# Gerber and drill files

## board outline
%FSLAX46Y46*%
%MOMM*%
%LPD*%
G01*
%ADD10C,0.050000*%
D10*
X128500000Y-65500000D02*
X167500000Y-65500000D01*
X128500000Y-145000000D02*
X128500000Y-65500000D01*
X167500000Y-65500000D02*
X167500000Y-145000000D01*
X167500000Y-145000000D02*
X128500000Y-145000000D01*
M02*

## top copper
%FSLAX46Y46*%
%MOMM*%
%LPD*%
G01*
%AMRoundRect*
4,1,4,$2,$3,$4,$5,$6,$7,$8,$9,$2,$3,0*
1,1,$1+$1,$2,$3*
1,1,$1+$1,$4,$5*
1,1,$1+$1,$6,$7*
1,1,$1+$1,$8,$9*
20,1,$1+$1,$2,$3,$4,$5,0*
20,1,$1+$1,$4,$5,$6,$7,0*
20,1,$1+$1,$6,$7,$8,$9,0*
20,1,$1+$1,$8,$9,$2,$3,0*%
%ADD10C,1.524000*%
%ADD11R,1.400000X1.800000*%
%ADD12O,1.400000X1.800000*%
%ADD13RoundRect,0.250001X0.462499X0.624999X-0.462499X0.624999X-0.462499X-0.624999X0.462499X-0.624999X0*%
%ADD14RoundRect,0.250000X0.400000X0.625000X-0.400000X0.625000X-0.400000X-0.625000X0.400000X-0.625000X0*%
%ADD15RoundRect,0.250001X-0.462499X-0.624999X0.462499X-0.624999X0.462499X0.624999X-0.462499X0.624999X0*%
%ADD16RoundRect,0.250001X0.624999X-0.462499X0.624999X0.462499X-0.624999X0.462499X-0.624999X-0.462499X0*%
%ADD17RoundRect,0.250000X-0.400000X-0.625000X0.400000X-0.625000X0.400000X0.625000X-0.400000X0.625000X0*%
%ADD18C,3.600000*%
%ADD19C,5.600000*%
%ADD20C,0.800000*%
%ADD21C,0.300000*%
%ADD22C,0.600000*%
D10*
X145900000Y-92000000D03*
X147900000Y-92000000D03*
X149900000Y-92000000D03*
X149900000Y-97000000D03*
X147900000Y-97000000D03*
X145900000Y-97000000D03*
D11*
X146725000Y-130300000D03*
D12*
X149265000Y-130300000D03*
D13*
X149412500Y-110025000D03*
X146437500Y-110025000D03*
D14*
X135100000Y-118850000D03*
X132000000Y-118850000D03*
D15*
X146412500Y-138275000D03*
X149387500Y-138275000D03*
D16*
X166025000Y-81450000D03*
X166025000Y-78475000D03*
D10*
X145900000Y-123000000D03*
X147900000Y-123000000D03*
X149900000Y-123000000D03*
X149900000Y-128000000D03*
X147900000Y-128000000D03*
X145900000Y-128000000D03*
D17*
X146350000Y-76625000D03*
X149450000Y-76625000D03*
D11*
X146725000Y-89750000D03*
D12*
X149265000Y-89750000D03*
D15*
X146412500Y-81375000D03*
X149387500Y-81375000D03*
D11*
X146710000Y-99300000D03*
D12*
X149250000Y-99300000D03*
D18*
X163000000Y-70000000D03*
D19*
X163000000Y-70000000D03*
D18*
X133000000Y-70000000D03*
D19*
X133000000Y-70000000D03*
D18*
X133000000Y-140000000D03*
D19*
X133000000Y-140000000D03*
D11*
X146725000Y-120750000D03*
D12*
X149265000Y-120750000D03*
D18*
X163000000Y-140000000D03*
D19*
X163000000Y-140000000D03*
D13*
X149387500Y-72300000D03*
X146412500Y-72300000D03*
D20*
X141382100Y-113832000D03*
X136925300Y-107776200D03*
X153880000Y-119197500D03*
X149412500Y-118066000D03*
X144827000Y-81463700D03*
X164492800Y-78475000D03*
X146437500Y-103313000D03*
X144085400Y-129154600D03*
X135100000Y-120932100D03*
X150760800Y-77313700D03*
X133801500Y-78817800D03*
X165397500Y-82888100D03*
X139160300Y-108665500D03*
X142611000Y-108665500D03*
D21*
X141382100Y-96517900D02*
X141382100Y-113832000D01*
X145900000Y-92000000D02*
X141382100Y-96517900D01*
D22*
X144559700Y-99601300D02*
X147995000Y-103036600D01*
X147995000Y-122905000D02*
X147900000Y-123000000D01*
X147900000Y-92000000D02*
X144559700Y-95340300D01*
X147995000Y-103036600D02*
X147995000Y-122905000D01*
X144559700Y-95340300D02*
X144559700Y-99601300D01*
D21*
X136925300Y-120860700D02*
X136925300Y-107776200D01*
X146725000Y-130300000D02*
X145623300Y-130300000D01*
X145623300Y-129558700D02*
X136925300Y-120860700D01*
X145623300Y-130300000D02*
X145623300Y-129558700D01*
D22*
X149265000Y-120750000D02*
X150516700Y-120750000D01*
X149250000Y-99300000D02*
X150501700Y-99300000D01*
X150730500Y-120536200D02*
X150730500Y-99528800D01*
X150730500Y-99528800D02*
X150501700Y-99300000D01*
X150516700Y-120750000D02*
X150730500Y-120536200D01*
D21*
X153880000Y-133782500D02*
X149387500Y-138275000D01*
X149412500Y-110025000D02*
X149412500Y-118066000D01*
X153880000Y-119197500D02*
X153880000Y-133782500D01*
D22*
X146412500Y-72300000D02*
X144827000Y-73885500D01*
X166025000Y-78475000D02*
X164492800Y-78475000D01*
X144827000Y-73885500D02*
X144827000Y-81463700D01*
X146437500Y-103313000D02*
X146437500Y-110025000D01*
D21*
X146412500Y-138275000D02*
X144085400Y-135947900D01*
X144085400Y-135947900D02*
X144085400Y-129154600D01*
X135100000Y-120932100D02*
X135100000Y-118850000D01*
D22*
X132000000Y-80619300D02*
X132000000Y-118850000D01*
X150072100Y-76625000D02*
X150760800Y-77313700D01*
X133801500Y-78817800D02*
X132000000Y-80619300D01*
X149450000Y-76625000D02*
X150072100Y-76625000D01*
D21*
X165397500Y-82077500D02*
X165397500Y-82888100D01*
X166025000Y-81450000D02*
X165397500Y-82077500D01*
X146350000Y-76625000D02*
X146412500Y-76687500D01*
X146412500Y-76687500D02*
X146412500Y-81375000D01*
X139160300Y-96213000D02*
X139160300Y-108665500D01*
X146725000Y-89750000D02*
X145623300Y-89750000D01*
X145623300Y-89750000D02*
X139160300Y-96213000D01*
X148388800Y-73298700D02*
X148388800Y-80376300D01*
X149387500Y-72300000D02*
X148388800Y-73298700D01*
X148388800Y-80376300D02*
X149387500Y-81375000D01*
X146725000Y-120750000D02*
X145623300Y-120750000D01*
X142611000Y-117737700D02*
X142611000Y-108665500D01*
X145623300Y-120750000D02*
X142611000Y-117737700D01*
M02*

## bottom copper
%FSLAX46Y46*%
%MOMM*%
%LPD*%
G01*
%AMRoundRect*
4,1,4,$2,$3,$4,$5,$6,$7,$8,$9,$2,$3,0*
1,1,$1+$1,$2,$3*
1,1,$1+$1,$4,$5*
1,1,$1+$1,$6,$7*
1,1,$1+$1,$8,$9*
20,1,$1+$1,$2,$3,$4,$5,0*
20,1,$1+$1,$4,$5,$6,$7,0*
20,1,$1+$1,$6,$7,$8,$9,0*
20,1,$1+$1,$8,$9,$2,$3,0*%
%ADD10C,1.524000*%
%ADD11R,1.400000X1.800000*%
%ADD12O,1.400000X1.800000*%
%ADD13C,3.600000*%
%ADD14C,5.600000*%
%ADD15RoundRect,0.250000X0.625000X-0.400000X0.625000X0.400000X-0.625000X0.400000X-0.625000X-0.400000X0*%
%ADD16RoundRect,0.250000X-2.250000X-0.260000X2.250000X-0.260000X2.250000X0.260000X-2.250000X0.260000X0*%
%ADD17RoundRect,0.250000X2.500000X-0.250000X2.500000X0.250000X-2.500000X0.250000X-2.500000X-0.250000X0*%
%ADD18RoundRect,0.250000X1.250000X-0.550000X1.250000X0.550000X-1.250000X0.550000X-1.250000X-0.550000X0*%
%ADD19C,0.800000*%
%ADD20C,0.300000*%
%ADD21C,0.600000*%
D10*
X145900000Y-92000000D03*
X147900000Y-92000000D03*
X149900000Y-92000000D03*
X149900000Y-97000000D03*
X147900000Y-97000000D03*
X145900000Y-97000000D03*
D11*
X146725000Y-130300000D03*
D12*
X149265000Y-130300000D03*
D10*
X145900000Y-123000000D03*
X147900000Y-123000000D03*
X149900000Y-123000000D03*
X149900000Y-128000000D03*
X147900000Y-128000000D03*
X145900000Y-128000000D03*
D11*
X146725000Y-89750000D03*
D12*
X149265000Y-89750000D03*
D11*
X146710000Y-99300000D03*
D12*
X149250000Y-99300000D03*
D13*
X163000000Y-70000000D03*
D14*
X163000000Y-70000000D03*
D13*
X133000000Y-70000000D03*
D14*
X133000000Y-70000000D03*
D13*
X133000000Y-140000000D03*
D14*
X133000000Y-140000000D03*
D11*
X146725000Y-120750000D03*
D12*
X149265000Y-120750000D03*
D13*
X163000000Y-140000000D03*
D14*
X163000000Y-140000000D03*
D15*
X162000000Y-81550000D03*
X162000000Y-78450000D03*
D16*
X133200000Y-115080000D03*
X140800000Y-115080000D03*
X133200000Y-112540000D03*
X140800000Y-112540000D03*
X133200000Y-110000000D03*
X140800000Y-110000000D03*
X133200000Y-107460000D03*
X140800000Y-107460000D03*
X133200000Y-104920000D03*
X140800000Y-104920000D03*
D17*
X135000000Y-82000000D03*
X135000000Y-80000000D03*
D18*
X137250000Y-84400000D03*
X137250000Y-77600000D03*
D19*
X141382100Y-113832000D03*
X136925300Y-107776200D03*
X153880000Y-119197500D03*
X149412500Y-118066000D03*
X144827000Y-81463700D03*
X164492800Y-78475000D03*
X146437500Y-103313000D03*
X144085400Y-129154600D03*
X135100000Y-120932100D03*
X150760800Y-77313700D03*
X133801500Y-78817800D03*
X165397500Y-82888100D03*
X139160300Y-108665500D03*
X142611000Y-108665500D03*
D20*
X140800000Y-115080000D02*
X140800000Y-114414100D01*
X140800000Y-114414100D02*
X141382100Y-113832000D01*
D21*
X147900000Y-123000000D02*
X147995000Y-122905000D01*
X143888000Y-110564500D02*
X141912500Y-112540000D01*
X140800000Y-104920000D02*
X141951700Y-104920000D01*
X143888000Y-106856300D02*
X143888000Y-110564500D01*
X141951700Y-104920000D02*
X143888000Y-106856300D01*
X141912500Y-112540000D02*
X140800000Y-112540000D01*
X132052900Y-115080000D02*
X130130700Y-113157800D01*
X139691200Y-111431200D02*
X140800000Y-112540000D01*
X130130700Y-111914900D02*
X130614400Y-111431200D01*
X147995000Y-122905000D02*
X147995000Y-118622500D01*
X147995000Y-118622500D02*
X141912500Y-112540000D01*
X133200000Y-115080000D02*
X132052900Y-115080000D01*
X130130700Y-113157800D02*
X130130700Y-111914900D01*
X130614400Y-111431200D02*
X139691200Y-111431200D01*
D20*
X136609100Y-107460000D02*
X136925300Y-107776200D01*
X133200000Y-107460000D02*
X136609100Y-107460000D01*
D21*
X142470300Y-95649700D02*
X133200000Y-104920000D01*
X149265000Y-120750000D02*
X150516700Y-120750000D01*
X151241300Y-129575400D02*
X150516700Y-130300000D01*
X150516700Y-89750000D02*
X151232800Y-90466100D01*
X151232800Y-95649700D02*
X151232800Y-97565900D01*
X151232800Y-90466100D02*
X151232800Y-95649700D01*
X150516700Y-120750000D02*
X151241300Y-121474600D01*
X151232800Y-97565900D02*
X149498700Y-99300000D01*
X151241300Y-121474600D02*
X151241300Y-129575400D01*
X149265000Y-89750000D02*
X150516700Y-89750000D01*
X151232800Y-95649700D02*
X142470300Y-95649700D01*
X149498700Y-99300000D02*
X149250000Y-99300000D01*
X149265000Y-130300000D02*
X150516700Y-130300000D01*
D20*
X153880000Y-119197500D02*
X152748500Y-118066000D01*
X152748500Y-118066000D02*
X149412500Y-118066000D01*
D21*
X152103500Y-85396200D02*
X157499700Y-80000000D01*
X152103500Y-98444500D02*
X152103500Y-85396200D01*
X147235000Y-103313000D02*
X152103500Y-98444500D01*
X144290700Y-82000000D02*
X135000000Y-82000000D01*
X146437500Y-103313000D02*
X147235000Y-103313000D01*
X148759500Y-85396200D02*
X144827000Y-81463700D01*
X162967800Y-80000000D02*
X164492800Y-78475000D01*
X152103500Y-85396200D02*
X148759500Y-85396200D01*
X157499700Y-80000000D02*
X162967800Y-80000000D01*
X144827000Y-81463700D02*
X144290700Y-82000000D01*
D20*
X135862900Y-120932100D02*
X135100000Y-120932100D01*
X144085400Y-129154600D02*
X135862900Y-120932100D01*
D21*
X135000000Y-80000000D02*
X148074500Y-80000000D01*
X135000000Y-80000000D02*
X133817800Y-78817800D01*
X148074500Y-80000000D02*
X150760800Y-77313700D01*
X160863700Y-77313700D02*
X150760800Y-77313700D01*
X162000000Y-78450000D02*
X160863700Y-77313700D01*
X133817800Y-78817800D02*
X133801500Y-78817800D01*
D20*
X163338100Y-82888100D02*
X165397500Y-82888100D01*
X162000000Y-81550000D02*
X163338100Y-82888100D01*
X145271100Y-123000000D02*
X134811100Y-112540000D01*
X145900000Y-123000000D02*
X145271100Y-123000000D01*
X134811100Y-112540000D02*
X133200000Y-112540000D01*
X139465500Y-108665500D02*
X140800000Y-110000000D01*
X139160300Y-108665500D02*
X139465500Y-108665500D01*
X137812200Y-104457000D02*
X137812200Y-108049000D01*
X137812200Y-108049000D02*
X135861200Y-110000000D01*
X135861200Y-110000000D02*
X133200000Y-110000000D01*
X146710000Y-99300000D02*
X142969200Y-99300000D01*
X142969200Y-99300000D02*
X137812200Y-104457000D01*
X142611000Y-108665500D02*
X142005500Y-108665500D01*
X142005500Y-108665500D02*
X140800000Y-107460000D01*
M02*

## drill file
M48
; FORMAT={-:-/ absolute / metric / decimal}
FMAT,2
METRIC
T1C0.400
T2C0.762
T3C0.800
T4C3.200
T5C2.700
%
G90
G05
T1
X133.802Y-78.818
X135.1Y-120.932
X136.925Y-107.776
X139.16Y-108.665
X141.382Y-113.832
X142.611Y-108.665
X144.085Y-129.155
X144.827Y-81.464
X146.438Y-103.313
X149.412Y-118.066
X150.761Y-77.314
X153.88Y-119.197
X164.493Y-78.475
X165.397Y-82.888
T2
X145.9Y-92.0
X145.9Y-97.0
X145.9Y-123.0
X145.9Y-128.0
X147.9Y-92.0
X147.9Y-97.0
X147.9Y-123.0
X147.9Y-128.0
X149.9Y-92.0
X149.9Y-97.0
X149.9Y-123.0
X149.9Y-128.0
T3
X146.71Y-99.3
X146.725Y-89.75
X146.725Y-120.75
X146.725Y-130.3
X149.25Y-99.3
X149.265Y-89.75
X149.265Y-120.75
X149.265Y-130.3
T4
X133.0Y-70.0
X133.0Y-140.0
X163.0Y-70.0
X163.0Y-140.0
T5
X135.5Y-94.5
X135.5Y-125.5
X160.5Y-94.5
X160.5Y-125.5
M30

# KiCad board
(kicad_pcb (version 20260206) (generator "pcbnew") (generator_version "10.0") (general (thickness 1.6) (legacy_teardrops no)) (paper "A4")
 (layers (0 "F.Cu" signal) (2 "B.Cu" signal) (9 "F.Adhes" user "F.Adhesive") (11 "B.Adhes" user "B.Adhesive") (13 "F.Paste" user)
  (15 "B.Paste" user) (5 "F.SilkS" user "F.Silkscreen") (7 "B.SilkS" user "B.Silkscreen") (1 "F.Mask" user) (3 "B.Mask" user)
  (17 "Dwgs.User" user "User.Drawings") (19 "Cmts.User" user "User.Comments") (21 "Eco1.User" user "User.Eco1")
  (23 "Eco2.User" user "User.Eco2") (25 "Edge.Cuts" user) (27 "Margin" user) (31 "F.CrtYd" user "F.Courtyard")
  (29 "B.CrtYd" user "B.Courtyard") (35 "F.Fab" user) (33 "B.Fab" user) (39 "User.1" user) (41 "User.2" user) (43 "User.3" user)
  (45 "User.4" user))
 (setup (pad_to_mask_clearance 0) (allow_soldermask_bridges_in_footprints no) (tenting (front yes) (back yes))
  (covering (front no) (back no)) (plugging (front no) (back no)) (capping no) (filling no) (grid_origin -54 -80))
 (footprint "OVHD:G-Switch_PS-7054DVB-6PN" (layer "F.Cu") (at 148.5 100)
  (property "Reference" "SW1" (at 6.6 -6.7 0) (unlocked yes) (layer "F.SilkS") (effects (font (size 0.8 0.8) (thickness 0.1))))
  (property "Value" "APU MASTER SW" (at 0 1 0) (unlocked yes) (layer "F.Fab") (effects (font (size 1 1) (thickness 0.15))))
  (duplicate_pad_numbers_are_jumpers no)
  (pad "1" thru_hole circle (at -2.6 -8) (size 1.524 1.524) (drill 0.762) (layers "*.Cu" "*.Mask") (remove_unused_layers no)
   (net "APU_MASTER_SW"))
  (pad "2" thru_hole circle (at -0.6 -8) (size 1.524 1.524) (drill 0.762) (layers "*.Cu" "*.Mask") (remove_unused_layers no) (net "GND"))
  (pad "3" thru_hole circle (at 1.4 -8) (size 1.524 1.524) (drill 0.762) (layers "*.Cu" "*.Mask") (remove_unused_layers no)
   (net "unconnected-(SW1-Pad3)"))
  (pad "4" thru_hole circle (at 1.4 -3) (size 1.524 1.524) (drill 0.762) (layers "*.Cu" "*.Mask") (remove_unused_layers no)
   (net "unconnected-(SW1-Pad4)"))
  (pad "5" thru_hole circle (at -0.6 -3) (size 1.524 1.524) (drill 0.762) (layers "*.Cu" "*.Mask") (remove_unused_layers no)
   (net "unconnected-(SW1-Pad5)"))
  (pad "6" thru_hole circle (at -2.6 -3) (size 1.524 1.524) (drill 0.762) (layers "*.Cu" "*.Mask") (remove_unused_layers no)
   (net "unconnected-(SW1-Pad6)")))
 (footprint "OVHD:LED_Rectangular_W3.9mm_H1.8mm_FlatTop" (layer "F.Cu") (at 146.725 130.3)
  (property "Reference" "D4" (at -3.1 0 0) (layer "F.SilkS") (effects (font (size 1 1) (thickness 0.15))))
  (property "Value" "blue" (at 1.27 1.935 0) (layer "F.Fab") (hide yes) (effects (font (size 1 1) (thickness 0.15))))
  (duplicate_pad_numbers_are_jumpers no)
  (pad "1" thru_hole rect (at 0 0) (size 1.4 1.8) (drill 0.8) (layers "*.Cu" "*.Mask") (remove_unused_layers no) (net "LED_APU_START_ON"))
  (pad "2" thru_hole oval (at 2.54 0) (size 1.4 1.8) (drill 0.8) (layers "*.Cu" "*.Mask") (remove_unused_layers no) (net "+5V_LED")))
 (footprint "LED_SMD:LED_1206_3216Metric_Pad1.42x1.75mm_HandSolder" (layer "F.Cu") (at 147.925 110.025 180)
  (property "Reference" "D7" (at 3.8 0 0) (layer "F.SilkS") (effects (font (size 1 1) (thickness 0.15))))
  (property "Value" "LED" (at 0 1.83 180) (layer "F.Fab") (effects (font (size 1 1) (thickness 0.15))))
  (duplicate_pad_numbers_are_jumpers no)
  (pad "1" smd roundrect (at -1.4875 0 180) (size 1.425 1.75) (layers "F.Cu" "F.Mask" "F.Paste") (roundrect_rratio 0.175439) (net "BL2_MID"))
  (pad "2" smd roundrect (at 1.4875 0 180) (size 1.425 1.75) (layers "F.Cu" "F.Mask" "F.Paste") (roundrect_rratio 0.175439) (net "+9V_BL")))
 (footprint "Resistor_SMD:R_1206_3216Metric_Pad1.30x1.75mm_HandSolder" (layer "F.Cu") (at 133.55 118.85 180)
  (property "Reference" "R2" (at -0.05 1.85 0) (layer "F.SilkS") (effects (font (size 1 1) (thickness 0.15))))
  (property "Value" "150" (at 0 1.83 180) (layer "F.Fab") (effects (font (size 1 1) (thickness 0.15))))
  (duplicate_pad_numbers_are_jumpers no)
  (pad "1" smd roundrect (at -1.55 0 180) (size 1.3 1.75) (layers "F.Cu" "F.Mask" "F.Paste") (roundrect_rratio 0.192308) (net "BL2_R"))
  (pad "2" smd roundrect (at 1.55 0 180) (size 1.3 1.75) (layers "F.Cu" "F.Mask" "F.Paste") (roundrect_rratio 0.192308) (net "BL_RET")))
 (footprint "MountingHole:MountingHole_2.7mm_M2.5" (layer "F.Cu") (at 135.5 125.5)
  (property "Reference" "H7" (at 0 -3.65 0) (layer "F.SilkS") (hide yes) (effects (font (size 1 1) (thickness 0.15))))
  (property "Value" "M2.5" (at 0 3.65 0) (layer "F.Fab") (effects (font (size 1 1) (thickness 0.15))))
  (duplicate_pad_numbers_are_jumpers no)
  (pad "" np_thru_hole circle (at 0 0) (size 2.7 2.7) (drill 2.7) (layers "*.Cu" "*.Mask")))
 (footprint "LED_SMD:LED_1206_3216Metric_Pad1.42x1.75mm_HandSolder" (layer "F.Cu") (at 147.9 138.275)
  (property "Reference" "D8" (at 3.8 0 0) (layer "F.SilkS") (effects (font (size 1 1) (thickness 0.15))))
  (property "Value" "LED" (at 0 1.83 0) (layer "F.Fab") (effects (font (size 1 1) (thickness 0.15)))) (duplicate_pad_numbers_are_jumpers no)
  (pad "1" smd roundrect (at -1.4875 0) (size 1.425 1.75) (layers "F.Cu" "F.Mask" "F.Paste") (roundrect_rratio 0.175439) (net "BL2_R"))
  (pad "2" smd roundrect (at 1.4875 0) (size 1.425 1.75) (layers "F.Cu" "F.Mask" "F.Paste") (roundrect_rratio 0.175439) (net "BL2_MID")))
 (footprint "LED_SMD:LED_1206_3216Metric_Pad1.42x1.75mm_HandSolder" (layer "F.Cu") (at 166.025 79.9625 90)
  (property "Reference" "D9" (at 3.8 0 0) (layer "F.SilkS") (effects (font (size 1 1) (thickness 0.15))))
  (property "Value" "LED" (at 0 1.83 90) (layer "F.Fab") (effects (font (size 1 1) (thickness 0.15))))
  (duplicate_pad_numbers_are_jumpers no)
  (pad "1" smd roundrect (at -1.4875 0 90) (size 1.425 1.75) (layers "F.Cu" "F.Mask" "F.Paste") (roundrect_rratio 0.175439) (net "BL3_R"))
  (pad "2" smd roundrect (at 1.4875 0 90) (size 1.425 1.75) (layers "F.Cu" "F.Mask" "F.Paste") (roundrect_rratio 0.175439) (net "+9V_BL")))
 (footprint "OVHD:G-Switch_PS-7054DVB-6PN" (layer "F.Cu") (at 148.5 131)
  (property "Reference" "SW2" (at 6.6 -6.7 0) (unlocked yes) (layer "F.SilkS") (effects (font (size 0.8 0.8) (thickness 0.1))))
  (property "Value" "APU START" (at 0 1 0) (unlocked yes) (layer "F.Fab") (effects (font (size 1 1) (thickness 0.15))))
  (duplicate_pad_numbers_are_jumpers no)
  (pad "1" thru_hole circle (at -2.6 -8) (size 1.524 1.524) (drill 0.762) (layers "*.Cu" "*.Mask") (remove_unused_layers no)
   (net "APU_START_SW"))
  (pad "2" thru_hole circle (at -0.6 -8) (size 1.524 1.524) (drill 0.762) (layers "*.Cu" "*.Mask") (remove_unused_layers no) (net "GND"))
  (pad "3" thru_hole circle (at 1.4 -8) (size 1.524 1.524) (drill 0.762) (layers "*.Cu" "*.Mask") (remove_unused_layers no)
   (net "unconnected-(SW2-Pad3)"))
  (pad "4" thru_hole circle (at 1.4 -3) (size 1.524 1.524) (drill 0.762) (layers "*.Cu" "*.Mask") (remove_unused_layers no)
   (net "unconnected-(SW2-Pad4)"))
  (pad "5" thru_hole circle (at -0.6 -3) (size 1.524 1.524) (drill 0.762) (layers "*.Cu" "*.Mask") (remove_unused_layers no)
   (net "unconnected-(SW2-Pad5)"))
  (pad "6" thru_hole circle (at -2.6 -3) (size 1.524 1.524) (drill 0.762) (layers "*.Cu" "*.Mask") (remove_unused_layers no)
   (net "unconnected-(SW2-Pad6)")))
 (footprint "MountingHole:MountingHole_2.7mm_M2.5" (layer "F.Cu") (at 135.5 94.5)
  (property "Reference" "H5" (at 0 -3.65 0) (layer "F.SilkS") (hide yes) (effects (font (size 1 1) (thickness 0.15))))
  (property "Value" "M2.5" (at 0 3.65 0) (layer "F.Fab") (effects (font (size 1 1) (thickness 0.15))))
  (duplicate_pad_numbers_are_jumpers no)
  (pad "" np_thru_hole circle (at 0 0) (size 2.7 2.7) (drill 2.7) (layers "*.Cu" "*.Mask")))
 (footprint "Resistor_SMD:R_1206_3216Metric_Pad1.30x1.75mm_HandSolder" (layer "F.Cu") (at 147.9 76.625)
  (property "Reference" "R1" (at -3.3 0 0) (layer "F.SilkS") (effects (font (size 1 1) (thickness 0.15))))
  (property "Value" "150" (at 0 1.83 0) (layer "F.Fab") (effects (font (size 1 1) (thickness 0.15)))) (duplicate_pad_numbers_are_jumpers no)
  (pad "1" smd roundrect (at -1.55 0) (size 1.3 1.75) (layers "F.Cu" "F.Mask" "F.Paste") (roundrect_rratio 0.192308) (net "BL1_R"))
  (pad "2" smd roundrect (at 1.55 0) (size 1.3 1.75) (layers "F.Cu" "F.Mask" "F.Paste") (roundrect_rratio 0.192308) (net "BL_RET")))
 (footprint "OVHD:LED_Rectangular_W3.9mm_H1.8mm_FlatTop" (layer "F.Cu") (at 146.725 89.75)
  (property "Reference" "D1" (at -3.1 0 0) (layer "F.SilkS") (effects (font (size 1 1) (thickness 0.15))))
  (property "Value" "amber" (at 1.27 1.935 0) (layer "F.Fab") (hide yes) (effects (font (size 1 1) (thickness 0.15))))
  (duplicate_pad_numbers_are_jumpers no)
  (pad "1" thru_hole rect (at 0 0) (size 1.4 1.8) (drill 0.8) (layers "*.Cu" "*.Mask") (remove_unused_layers no)
   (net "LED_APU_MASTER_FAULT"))
  (pad "2" thru_hole oval (at 2.54 0) (size 1.4 1.8) (drill 0.8) (layers "*.Cu" "*.Mask") (remove_unused_layers no) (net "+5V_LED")))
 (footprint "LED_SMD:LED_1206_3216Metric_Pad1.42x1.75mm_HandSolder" (layer "F.Cu") (at 147.9 81.375)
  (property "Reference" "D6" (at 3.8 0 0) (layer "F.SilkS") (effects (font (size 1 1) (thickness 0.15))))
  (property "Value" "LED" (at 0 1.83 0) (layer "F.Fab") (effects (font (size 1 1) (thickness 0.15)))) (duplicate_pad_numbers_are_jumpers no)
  (pad "1" smd roundrect (at -1.4875 0) (size 1.425 1.75) (layers "F.Cu" "F.Mask" "F.Paste") (roundrect_rratio 0.175439) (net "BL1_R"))
  (pad "2" smd roundrect (at 1.4875 0) (size 1.425 1.75) (layers "F.Cu" "F.Mask" "F.Paste") (roundrect_rratio 0.175439) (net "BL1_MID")))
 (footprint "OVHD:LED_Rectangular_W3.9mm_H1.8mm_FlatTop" (layer "F.Cu") (at 146.71 99.3)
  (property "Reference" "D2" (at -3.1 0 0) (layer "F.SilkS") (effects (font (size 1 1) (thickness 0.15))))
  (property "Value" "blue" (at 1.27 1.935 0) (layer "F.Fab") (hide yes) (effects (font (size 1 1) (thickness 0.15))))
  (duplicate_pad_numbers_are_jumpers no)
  (pad "1" thru_hole rect (at 0 0) (size 1.4 1.8) (drill 0.8) (layers "*.Cu" "*.Mask") (remove_unused_layers no) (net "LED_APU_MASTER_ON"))
  (pad "2" thru_hole oval (at 2.54 0) (size 1.4 1.8) (drill 0.8) (layers "*.Cu" "*.Mask") (remove_unused_layers no) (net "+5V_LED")))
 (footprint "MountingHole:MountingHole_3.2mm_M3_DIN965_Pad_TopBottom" (layer "F.Cu") (at 163 70)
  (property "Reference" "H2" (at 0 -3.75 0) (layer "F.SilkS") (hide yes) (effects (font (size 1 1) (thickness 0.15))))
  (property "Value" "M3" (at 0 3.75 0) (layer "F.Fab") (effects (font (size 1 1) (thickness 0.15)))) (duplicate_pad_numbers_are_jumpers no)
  (pad "1" thru_hole circle (at 0 0) (size 3.6 3.6) (drill 3.2) (layers "*.Cu" "*.Mask") (remove_unused_layers no)
   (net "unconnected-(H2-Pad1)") (zone_connect 2))
  (pad "1" connect circle (at 0 0) (size 5.6 5.6) (layers "F.Cu" "F.Mask") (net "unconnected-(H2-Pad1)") (zone_connect 2))
  (pad "1" connect circle (at 0 0) (size 5.6 5.6) (layers "B.Cu" "B.Mask") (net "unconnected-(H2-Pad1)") (zone_connect 2)))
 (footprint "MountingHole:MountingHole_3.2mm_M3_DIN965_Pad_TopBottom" (layer "F.Cu") (at 133 70)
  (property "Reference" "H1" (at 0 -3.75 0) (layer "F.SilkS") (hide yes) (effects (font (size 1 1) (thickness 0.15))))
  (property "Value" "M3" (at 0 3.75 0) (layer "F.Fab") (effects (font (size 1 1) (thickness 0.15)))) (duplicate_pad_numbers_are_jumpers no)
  (pad "1" thru_hole circle (at 0 0) (size 3.6 3.6) (drill 3.2) (layers "*.Cu" "*.Mask") (remove_unused_layers no)
   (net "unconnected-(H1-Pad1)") (zone_connect 2))
  (pad "1" connect circle (at 0 0) (size 5.6 5.6) (layers "F.Cu" "F.Mask") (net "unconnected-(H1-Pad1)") (zone_connect 2))
  (pad "1" connect circle (at 0 0) (size 5.6 5.6) (layers "B.Cu" "B.Mask") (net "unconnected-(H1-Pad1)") (zone_connect 2)))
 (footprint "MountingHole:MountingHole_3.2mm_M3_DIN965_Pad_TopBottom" (layer "F.Cu") (at 133 140)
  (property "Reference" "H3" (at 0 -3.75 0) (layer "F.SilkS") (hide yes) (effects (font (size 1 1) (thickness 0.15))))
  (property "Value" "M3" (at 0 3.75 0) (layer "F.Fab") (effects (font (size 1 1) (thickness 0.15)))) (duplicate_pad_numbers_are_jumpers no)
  (pad "1" thru_hole circle (at 0 0) (size 3.6 3.6) (drill 3.2) (layers "*.Cu" "*.Mask") (remove_unused_layers no)
   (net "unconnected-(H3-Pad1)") (zone_connect 2))
  (pad "1" connect circle (at 0 0) (size 5.6 5.6) (layers "F.Cu" "F.Mask") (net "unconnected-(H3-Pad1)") (zone_connect 2))
  (pad "1" connect circle (at 0 0) (size 5.6 5.6) (layers "B.Cu" "B.Mask") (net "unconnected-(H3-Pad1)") (zone_connect 2)))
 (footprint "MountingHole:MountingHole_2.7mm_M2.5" (layer "F.Cu") (at 160.5 125.5)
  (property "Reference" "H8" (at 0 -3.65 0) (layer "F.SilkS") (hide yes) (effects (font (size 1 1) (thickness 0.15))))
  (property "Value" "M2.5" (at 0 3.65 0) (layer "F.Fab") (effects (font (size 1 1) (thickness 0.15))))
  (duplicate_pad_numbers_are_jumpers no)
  (pad "" np_thru_hole circle (at 0 0) (size 2.7 2.7) (drill 2.7) (layers "*.Cu" "*.Mask")))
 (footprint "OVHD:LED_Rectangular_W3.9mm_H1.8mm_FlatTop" (layer "F.Cu") (at 146.725 120.75)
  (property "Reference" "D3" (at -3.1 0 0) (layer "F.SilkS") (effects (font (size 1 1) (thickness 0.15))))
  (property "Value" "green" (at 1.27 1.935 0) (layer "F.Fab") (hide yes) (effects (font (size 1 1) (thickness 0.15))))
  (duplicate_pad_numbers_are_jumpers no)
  (pad "1" thru_hole rect (at 0 0) (size 1.4 1.8) (drill 0.8) (layers "*.Cu" "*.Mask") (remove_unused_layers no) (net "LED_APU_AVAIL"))
  (pad "2" thru_hole oval (at 2.54 0) (size 1.4 1.8) (drill 0.8) (layers "*.Cu" "*.Mask") (remove_unused_layers no) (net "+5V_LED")))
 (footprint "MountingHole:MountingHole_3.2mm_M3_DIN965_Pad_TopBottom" (layer "F.Cu") (at 163 140)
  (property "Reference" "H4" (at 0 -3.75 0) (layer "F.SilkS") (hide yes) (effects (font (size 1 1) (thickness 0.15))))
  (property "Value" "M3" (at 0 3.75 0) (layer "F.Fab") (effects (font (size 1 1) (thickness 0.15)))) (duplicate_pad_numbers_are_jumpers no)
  (pad "1" thru_hole circle (at 0 0) (size 3.6 3.6) (drill 3.2) (layers "*.Cu" "*.Mask") (remove_unused_layers no)
   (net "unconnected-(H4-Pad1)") (zone_connect 2))
  (pad "1" connect circle (at 0 0) (size 5.6 5.6) (layers "F.Cu" "F.Mask") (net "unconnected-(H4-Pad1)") (zone_connect 2))
  (pad "1" connect circle (at 0 0) (size 5.6 5.6) (layers "B.Cu" "B.Mask") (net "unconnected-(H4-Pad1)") (zone_connect 2)))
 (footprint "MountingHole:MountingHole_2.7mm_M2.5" (layer "F.Cu") (at 160.5 94.5)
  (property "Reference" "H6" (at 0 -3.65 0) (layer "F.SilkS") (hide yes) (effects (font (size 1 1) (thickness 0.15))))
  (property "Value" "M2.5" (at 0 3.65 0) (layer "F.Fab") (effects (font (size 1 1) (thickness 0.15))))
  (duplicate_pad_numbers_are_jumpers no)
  (pad "" np_thru_hole circle (at 0 0) (size 2.7 2.7) (drill 2.7) (layers "*.Cu" "*.Mask")))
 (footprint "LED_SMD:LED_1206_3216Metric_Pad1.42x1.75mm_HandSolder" (layer "F.Cu") (at 147.9 72.3 180)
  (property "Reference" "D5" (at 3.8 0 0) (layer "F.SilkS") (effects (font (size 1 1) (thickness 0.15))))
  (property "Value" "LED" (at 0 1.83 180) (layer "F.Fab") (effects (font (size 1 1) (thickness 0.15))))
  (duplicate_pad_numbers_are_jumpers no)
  (pad "1" smd roundrect (at -1.4875 0 180) (size 1.425 1.75) (layers "F.Cu" "F.Mask" "F.Paste") (roundrect_rratio 0.175439) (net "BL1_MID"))
  (pad "2" smd roundrect (at 1.4875 0 180) (size 1.425 1.75) (layers "F.Cu" "F.Mask" "F.Paste") (roundrect_rratio 0.175439) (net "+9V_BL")))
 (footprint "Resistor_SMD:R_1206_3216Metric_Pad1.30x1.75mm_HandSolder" (layer "B.Cu") (at 162 80 90)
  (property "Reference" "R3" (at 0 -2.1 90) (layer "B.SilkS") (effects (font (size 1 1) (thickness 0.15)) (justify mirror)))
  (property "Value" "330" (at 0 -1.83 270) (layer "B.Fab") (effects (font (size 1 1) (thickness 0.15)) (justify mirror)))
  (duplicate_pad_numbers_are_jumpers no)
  (pad "1" smd roundrect (at -1.55 0 90) (size 1.3 1.75) (layers "B.Cu" "B.Mask" "B.Paste") (roundrect_rratio 0.192308) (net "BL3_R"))
  (pad "2" smd roundrect (at 1.55 0 90) (size 1.3 1.75) (layers "B.Cu" "B.Mask" "B.Paste") (roundrect_rratio 0.192308) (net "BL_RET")))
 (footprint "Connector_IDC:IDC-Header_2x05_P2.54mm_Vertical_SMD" (layer "B.Cu") (at 137 110)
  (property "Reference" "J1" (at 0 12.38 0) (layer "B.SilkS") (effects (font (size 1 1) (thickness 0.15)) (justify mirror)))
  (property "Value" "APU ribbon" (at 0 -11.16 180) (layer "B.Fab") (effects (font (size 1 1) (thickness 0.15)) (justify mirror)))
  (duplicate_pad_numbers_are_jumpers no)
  (pad "1" smd roundrect (at -3.8 5.08) (size 5 1.02) (layers "B.Cu" "B.Mask" "B.Paste") (roundrect_rratio 0.245098) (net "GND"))
  (pad "2" smd roundrect (at 3.8 5.08) (size 5 1.02) (layers "B.Cu" "B.Mask" "B.Paste") (roundrect_rratio 0.245098) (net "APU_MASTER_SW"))
  (pad "3" smd roundrect (at -3.8 2.54) (size 5 1.02) (layers "B.Cu" "B.Mask" "B.Paste") (roundrect_rratio 0.245098) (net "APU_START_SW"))
  (pad "4" smd roundrect (at 3.8 2.54) (size 5 1.02) (layers "B.Cu" "B.Mask" "B.Paste") (roundrect_rratio 0.245098) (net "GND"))
  (pad "5" smd roundrect (at -3.8 0) (size 5 1.02) (layers "B.Cu" "B.Mask" "B.Paste") (roundrect_rratio 0.245098) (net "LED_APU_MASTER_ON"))
  (pad "6" smd roundrect (at 3.8 0) (size 5 1.02) (layers "B.Cu" "B.Mask" "B.Paste") (roundrect_rratio 0.245098)
   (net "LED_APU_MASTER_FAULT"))
  (pad "7" smd roundrect (at -3.8 -2.54) (size 5 1.02) (layers "B.Cu" "B.Mask" "B.Paste") (roundrect_rratio 0.245098)
   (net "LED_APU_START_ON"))
  (pad "8" smd roundrect (at 3.8 -2.54) (size 5 1.02) (layers "B.Cu" "B.Mask" "B.Paste") (roundrect_rratio 0.245098) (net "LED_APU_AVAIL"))
  (pad "9" smd roundrect (at -3.8 -5.08) (size 5 1.02) (layers "B.Cu" "B.Mask" "B.Paste") (roundrect_rratio 0.245098) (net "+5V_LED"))
  (pad "10" smd roundrect (at 3.8 -5.08) (size 5 1.02) (layers "B.Cu" "B.Mask" "B.Paste") (roundrect_rratio 0.245098) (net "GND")))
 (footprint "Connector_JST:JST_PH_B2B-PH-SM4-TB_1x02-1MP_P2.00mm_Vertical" (layer "B.Cu") (at 135.5 81 90)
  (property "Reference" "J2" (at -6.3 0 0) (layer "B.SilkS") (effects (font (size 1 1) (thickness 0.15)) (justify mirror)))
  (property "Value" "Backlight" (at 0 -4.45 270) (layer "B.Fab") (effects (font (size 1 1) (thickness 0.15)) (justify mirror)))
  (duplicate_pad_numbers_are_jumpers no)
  (pad "1" smd roundrect (at -1 -0.5 90) (size 1 5.5) (layers "B.Cu" "B.Mask" "B.Paste") (roundrect_rratio 0.25) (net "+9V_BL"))
  (pad "2" smd roundrect (at 1 -0.5 90) (size 1 5.5) (layers "B.Cu" "B.Mask" "B.Paste") (roundrect_rratio 0.25) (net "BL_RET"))
  (pad "MP" smd roundrect (at -3.4 1.75 90) (size 1.6 3) (layers "B.Cu" "B.Mask" "B.Paste") (roundrect_rratio 0.15625))
  (pad "MP" smd roundrect (at 3.4 1.75 90) (size 1.6 3) (layers "B.Cu" "B.Mask" "B.Paste") (roundrect_rratio 0.15625)))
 (gr_line (start 128.5 65.5) (end 167.5 65.5) (stroke (width 0.05) (type default)) (layer "Edge.Cuts"))
 (gr_line (start 128.5 145) (end 128.5 65.5) (stroke (width 0.05) (type default)) (layer "Edge.Cuts"))
 (gr_line (start 167.5 65.5) (end 167.5 145) (stroke (width 0.05) (type default)) (layer "Edge.Cuts"))
 (gr_line (start 167.5 145) (end 128.5 145) (stroke (width 0.05) (type default)) (layer "Edge.Cuts"))
 (segment (start 141.3821 96.5179) (end 141.3821 113.832) (width 0.3) (layer "F.Cu") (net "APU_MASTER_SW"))
 (segment (start 145.9 92) (end 141.3821 96.5179) (width 0.3) (layer "F.Cu") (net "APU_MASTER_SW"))
 (via (at 141.3821 113.832) (size 0.8) (drill 0.4) (layers "F.Cu" "B.Cu") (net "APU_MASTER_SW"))
 (segment (start 140.8 115.08) (end 140.8 114.4141) (width 0.3) (layer "B.Cu") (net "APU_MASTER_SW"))
 (segment (start 140.8 114.4141) (end 141.3821 113.832) (width 0.3) (layer "B.Cu") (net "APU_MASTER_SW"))
 (segment (start 144.5597 99.6013) (end 147.995 103.0366) (width 0.6) (layer "F.Cu") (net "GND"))
 (segment (start 147.995 122.905) (end 147.9 123) (width 0.6) (layer "F.Cu") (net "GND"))
 (segment (start 147.9 92) (end 144.5597 95.3403) (width 0.6) (layer "F.Cu") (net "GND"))
 (segment (start 147.995 103.0366) (end 147.995 122.905) (width 0.6) (layer "F.Cu") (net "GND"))
 (segment (start 144.5597 95.3403) (end 144.5597 99.6013) (width 0.6) (layer "F.Cu") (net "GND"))
 (segment (start 147.9 123) (end 147.995 122.905) (width 0.6) (layer "B.Cu") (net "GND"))
 (segment (start 143.888 110.5645) (end 141.9125 112.54) (width 0.6) (layer "B.Cu") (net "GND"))
 (segment (start 140.8 104.92) (end 141.9517 104.92) (width 0.6) (layer "B.Cu") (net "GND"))
 (segment (start 143.888 106.8563) (end 143.888 110.5645) (width 0.6) (layer "B.Cu") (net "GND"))
 (segment (start 141.9517 104.92) (end 143.888 106.8563) (width 0.6) (layer "B.Cu") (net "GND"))
 (segment (start 141.9125 112.54) (end 140.8 112.54) (width 0.6) (layer "B.Cu") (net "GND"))
 (segment (start 132.0529 115.08) (end 130.1307 113.1578) (width 0.6) (layer "B.Cu") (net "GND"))
 (segment (start 139.6912 111.4312) (end 140.8 112.54) (width 0.6) (layer "B.Cu") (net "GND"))
 (segment (start 130.1307 111.9149) (end 130.6144 111.4312) (width 0.6) (layer "B.Cu") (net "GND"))
 (segment (start 147.995 122.905) (end 147.995 118.6225) (width 0.6) (layer "B.Cu") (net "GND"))
 (segment (start 147.995 118.6225) (end 141.9125 112.54) (width 0.6) (layer "B.Cu") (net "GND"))
 (segment (start 133.2 115.08) (end 132.0529 115.08) (width 0.6) (layer "B.Cu") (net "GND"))
 (segment (start 130.1307 113.1578) (end 130.1307 111.9149) (width 0.6) (layer "B.Cu") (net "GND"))
 (segment (start 130.6144 111.4312) (end 139.6912 111.4312) (width 0.6) (layer "B.Cu") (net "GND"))
 (segment (start 136.9253 120.8607) (end 136.9253 107.7762) (width 0.3) (layer "F.Cu") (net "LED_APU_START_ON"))
 (segment (start 146.725 130.3) (end 145.6233 130.3) (width 0.3) (layer "F.Cu") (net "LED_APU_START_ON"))
 (segment (start 145.6233 129.5587) (end 136.9253 120.8607) (width 0.3) (layer "F.Cu") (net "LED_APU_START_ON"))
 (segment (start 145.6233 130.3) (end 145.6233 129.5587) (width 0.3) (layer "F.Cu") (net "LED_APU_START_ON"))
 (via (at 136.9253 107.7762) (size 0.8) (drill 0.4) (layers "F.Cu" "B.Cu") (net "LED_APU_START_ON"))
 (segment (start 136.6091 107.46) (end 136.9253 107.7762) (width 0.3) (layer "B.Cu") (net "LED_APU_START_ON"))
 (segment (start 133.2 107.46) (end 136.6091 107.46) (width 0.3) (layer "B.Cu") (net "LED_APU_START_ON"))
 (segment (start 149.265 120.75) (end 150.5167 120.75) (width 0.6) (layer "F.Cu") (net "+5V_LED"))
 (segment (start 149.25 99.3) (end 150.5017 99.3) (width 0.6) (layer "F.Cu") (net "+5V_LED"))
 (segment (start 150.7305 120.5362) (end 150.7305 99.5288) (width 0.6) (layer "F.Cu") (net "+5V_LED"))
 (segment (start 150.7305 99.5288) (end 150.5017 99.3) (width 0.6) (layer "F.Cu") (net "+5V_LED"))
 (segment (start 150.5167 120.75) (end 150.7305 120.5362) (width 0.6) (layer "F.Cu") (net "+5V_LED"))
 (segment (start 142.4703 95.6497) (end 133.2 104.92) (width 0.6) (layer "B.Cu") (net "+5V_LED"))
 (segment (start 149.265 120.75) (end 150.5167 120.75) (width 0.6) (layer "B.Cu") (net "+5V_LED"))
 (segment (start 151.2413 129.5754) (end 150.5167 130.3) (width 0.6) (layer "B.Cu") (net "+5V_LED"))
 (segment (start 150.5167 89.75) (end 151.2328 90.4661) (width 0.6) (layer "B.Cu") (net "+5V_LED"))
 (segment (start 151.2328 95.6497) (end 151.2328 97.5659) (width 0.6) (layer "B.Cu") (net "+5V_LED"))
 (segment (start 151.2328 90.4661) (end 151.2328 95.6497) (width 0.6) (layer "B.Cu") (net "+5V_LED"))
 (segment (start 150.5167 120.75) (end 151.2413 121.4746) (width 0.6) (layer "B.Cu") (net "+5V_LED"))
 (segment (start 151.2328 97.5659) (end 149.4987 99.3) (width 0.6) (layer "B.Cu") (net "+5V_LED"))
 (segment (start 151.2413 121.4746) (end 151.2413 129.5754) (width 0.6) (layer "B.Cu") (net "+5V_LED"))
 (segment (start 149.265 89.75) (end 150.5167 89.75) (width 0.6) (layer "B.Cu") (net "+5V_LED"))
 (segment (start 151.2328 95.6497) (end 142.4703 95.6497) (width 0.6) (layer "B.Cu") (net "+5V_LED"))
 (segment (start 149.4987 99.3) (end 149.25 99.3) (width 0.6) (layer "B.Cu") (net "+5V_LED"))
 (segment (start 149.265 130.3) (end 150.5167 130.3) (width 0.6) (layer "B.Cu") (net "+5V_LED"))
 (segment (start 153.88 133.7825) (end 149.3875 138.275) (width 0.3) (layer "F.Cu") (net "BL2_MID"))
 (segment (start 149.4125 110.025) (end 149.4125 118.066) (width 0.3) (layer "F.Cu") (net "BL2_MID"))
 (segment (start 153.88 119.1975) (end 153.88 133.7825) (width 0.3) (layer "F.Cu") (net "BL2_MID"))
 (via (at 153.88 119.1975) (size 0.8) (drill 0.4) (layers "F.Cu" "B.Cu") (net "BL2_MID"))
 (via (at 149.4125 118.066) (size 0.8) (drill 0.4) (layers "F.Cu" "B.Cu") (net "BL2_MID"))
 (segment (start 153.88 119.1975) (end 152.7485 118.066) (width 0.3) (layer "B.Cu") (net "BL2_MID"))
 (segment (start 152.7485 118.066) (end 149.4125 118.066) (width 0.3) (layer "B.Cu") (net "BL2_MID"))
 (segment (start 146.4125 72.3) (end 144.827 73.8855) (width 0.6) (layer "F.Cu") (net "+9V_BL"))
 (segment (start 166.025 78.475) (end 164.4928 78.475) (width 0.6) (layer "F.Cu") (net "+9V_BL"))
 (segment (start 144.827 73.8855) (end 144.827 81.4637) (width 0.6) (layer "F.Cu") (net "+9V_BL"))
 (segment (start 146.4375 103.313) (end 146.4375 110.025) (width 0.6) (layer "F.Cu") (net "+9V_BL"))
 (via (at 144.827 81.4637) (size 0.8) (drill 0.4) (layers "F.Cu" "B.Cu") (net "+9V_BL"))
 (via (at 164.4928 78.475) (size 0.8) (drill 0.4) (layers "F.Cu" "B.Cu") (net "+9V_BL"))
 (via (at 146.4375 103.313) (size 0.8) (drill 0.4) (layers "F.Cu" "B.Cu") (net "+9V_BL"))
 (segment (start 152.1035 85.3962) (end 157.4997 80) (width 0.6) (layer "B.Cu") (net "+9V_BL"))
 (segment (start 152.1035 98.4445) (end 152.1035 85.3962) (width 0.6) (layer "B.Cu") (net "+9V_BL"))
 (segment (start 147.235 103.313) (end 152.1035 98.4445) (width 0.6) (layer "B.Cu") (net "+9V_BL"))
 (segment (start 144.2907 82) (end 135 82) (width 0.6) (layer "B.Cu") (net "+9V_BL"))
 (segment (start 146.4375 103.313) (end 147.235 103.313) (width 0.6) (layer "B.Cu") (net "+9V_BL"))
 (segment (start 148.7595 85.3962) (end 144.827 81.4637) (width 0.6) (layer "B.Cu") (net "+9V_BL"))
 (segment (start 162.9678 80) (end 164.4928 78.475) (width 0.6) (layer "B.Cu") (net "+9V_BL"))
 (segment (start 152.1035 85.3962) (end 148.7595 85.3962) (width 0.6) (layer "B.Cu") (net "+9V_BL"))
 (segment (start 157.4997 80) (end 162.9678 80) (width 0.6) (layer "B.Cu") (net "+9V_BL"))
 (segment (start 144.827 81.4637) (end 144.2907 82) (width 0.6) (layer "B.Cu") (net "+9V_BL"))
 (segment (start 146.4125 138.275) (end 144.0854 135.9479) (width 0.3) (layer "F.Cu") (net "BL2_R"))
 (segment (start 144.0854 135.9479) (end 144.0854 129.1546) (width 0.3) (layer "F.Cu") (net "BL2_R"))
 (segment (start 135.1 120.9321) (end 135.1 118.85) (width 0.3) (layer "F.Cu") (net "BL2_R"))
 (via (at 144.0854 129.1546) (size 0.8) (drill 0.4) (layers "F.Cu" "B.Cu") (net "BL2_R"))
 (via (at 135.1 120.9321) (size 0.8) (drill 0.4) (layers "F.Cu" "B.Cu") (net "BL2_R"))
 (segment (start 135.8629 120.9321) (end 135.1 120.9321) (width 0.3) (layer "B.Cu") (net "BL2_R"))
 (segment (start 144.0854 129.1546) (end 135.8629 120.9321) (width 0.3) (layer "B.Cu") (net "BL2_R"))
 (segment (start 132 80.6193) (end 132 118.85) (width 0.6) (layer "F.Cu") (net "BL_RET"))
 (segment (start 150.0721 76.625) (end 150.7608 77.3137) (width 0.6) (layer "F.Cu") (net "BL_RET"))
 (segment (start 133.8015 78.8178) (end 132 80.6193) (width 0.6) (layer "F.Cu") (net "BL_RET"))
 (segment (start 149.45 76.625) (end 150.0721 76.625) (width 0.6) (layer "F.Cu") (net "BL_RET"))
 (via (at 150.7608 77.3137) (size 0.8) (drill 0.4) (layers "F.Cu" "B.Cu") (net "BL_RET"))
 (via (at 133.8015 78.8178) (size 0.8) (drill 0.4) (layers "F.Cu" "B.Cu") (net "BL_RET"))
 (segment (start 135 80) (end 148.0745 80) (width 0.6) (layer "B.Cu") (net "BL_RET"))
 (segment (start 135 80) (end 133.8178 78.8178) (width 0.6) (layer "B.Cu") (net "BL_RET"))
 (segment (start 148.0745 80) (end 150.7608 77.3137) (width 0.6) (layer "B.Cu") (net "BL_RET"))
 (segment (start 160.8637 77.3137) (end 150.7608 77.3137) (width 0.6) (layer "B.Cu") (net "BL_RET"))
 (segment (start 162 78.45) (end 160.8637 77.3137) (width 0.6) (layer "B.Cu") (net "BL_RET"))
 (segment (start 133.8178 78.8178) (end 133.8015 78.8178) (width 0.6) (layer "B.Cu") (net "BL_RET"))
 (segment (start 165.3975 82.0775) (end 165.3975 82.8881) (width 0.3) (layer "F.Cu") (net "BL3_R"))
 (segment (start 166.025 81.45) (end 165.3975 82.0775) (width 0.3) (layer "F.Cu") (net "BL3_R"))
 (via (at 165.3975 82.8881) (size 0.8) (drill 0.4) (layers "F.Cu" "B.Cu") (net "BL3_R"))
 (segment (start 163.3381 82.8881) (end 165.3975 82.8881) (width 0.3) (layer "B.Cu") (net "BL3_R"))
 (segment (start 162 81.55) (end 163.3381 82.8881) (width 0.3) (layer "B.Cu") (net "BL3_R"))
 (segment (start 145.2711 123) (end 134.8111 112.54) (width 0.3) (layer "B.Cu") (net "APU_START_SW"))
 (segment (start 145.9 123) (end 145.2711 123) (width 0.3) (layer "B.Cu") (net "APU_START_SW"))
 (segment (start 134.8111 112.54) (end 133.2 112.54) (width 0.3) (layer "B.Cu") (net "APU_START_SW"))
 (segment (start 146.35 76.625) (end 146.4125 76.6875) (width 0.3) (layer "F.Cu") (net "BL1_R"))
 (segment (start 146.4125 76.6875) (end 146.4125 81.375) (width 0.3) (layer "F.Cu") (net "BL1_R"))
 (segment (start 139.1603 96.213) (end 139.1603 108.6655) (width 0.3) (layer "F.Cu") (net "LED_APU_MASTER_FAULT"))
 (segment (start 146.725 89.75) (end 145.6233 89.75) (width 0.3) (layer "F.Cu") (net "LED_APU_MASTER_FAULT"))
 (segment (start 145.6233 89.75) (end 139.1603 96.213) (width 0.3) (layer "F.Cu") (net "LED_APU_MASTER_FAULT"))
 (via (at 139.1603 108.6655) (size 0.8) (drill 0.4) (layers "F.Cu" "B.Cu") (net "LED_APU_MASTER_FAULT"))
 (segment (start 139.4655 108.6655) (end 140.8 110) (width 0.3) (layer "B.Cu") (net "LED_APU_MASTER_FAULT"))
 (segment (start 139.1603 108.6655) (end 139.4655 108.6655) (width 0.3) (layer "B.Cu") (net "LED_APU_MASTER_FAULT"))
 (segment (start 148.3888 73.2987) (end 148.3888 80.3763) (width 0.3) (layer "F.Cu") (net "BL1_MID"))
 (segment (start 149.3875 72.3) (end 148.3888 73.2987) (width 0.3) (layer "F.Cu") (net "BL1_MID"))
 (segment (start 148.3888 80.3763) (end 149.3875 81.375) (width 0.3) (layer "F.Cu") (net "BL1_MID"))
 (segment (start 137.8122 104.457) (end 137.8122 108.049) (width 0.3) (layer "B.Cu") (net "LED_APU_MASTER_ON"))
 (segment (start 137.8122 108.049) (end 135.8612 110) (width 0.3) (layer "B.Cu") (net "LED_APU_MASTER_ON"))
 (segment (start 135.8612 110) (end 133.2 110) (width 0.3) (layer "B.Cu") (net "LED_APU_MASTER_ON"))
 (segment (start 146.71 99.3) (end 142.9692 99.3) (width 0.3) (layer "B.Cu") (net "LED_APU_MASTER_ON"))
 (segment (start 142.9692 99.3) (end 137.8122 104.457) (width 0.3) (layer "B.Cu") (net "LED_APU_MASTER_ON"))
 (segment (start 146.725 120.75) (end 145.6233 120.75) (width 0.3) (layer "F.Cu") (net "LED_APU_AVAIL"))
 (segment (start 142.611 117.7377) (end 142.611 108.6655) (width 0.3) (layer "F.Cu") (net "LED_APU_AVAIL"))
 (segment (start 145.6233 120.75) (end 142.611 117.7377) (width 0.3) (layer "F.Cu") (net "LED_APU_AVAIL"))
 (via (at 142.611 108.6655) (size 0.8) (drill 0.4) (layers "F.Cu" "B.Cu") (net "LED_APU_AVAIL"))
 (segment (start 142.611 108.6655) (end 142.0055 108.6655) (width 0.3) (layer "B.Cu") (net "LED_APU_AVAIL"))
 (segment (start 142.0055 108.6655) (end 140.8 107.46) (width 0.3) (layer "B.Cu") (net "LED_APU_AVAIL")))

